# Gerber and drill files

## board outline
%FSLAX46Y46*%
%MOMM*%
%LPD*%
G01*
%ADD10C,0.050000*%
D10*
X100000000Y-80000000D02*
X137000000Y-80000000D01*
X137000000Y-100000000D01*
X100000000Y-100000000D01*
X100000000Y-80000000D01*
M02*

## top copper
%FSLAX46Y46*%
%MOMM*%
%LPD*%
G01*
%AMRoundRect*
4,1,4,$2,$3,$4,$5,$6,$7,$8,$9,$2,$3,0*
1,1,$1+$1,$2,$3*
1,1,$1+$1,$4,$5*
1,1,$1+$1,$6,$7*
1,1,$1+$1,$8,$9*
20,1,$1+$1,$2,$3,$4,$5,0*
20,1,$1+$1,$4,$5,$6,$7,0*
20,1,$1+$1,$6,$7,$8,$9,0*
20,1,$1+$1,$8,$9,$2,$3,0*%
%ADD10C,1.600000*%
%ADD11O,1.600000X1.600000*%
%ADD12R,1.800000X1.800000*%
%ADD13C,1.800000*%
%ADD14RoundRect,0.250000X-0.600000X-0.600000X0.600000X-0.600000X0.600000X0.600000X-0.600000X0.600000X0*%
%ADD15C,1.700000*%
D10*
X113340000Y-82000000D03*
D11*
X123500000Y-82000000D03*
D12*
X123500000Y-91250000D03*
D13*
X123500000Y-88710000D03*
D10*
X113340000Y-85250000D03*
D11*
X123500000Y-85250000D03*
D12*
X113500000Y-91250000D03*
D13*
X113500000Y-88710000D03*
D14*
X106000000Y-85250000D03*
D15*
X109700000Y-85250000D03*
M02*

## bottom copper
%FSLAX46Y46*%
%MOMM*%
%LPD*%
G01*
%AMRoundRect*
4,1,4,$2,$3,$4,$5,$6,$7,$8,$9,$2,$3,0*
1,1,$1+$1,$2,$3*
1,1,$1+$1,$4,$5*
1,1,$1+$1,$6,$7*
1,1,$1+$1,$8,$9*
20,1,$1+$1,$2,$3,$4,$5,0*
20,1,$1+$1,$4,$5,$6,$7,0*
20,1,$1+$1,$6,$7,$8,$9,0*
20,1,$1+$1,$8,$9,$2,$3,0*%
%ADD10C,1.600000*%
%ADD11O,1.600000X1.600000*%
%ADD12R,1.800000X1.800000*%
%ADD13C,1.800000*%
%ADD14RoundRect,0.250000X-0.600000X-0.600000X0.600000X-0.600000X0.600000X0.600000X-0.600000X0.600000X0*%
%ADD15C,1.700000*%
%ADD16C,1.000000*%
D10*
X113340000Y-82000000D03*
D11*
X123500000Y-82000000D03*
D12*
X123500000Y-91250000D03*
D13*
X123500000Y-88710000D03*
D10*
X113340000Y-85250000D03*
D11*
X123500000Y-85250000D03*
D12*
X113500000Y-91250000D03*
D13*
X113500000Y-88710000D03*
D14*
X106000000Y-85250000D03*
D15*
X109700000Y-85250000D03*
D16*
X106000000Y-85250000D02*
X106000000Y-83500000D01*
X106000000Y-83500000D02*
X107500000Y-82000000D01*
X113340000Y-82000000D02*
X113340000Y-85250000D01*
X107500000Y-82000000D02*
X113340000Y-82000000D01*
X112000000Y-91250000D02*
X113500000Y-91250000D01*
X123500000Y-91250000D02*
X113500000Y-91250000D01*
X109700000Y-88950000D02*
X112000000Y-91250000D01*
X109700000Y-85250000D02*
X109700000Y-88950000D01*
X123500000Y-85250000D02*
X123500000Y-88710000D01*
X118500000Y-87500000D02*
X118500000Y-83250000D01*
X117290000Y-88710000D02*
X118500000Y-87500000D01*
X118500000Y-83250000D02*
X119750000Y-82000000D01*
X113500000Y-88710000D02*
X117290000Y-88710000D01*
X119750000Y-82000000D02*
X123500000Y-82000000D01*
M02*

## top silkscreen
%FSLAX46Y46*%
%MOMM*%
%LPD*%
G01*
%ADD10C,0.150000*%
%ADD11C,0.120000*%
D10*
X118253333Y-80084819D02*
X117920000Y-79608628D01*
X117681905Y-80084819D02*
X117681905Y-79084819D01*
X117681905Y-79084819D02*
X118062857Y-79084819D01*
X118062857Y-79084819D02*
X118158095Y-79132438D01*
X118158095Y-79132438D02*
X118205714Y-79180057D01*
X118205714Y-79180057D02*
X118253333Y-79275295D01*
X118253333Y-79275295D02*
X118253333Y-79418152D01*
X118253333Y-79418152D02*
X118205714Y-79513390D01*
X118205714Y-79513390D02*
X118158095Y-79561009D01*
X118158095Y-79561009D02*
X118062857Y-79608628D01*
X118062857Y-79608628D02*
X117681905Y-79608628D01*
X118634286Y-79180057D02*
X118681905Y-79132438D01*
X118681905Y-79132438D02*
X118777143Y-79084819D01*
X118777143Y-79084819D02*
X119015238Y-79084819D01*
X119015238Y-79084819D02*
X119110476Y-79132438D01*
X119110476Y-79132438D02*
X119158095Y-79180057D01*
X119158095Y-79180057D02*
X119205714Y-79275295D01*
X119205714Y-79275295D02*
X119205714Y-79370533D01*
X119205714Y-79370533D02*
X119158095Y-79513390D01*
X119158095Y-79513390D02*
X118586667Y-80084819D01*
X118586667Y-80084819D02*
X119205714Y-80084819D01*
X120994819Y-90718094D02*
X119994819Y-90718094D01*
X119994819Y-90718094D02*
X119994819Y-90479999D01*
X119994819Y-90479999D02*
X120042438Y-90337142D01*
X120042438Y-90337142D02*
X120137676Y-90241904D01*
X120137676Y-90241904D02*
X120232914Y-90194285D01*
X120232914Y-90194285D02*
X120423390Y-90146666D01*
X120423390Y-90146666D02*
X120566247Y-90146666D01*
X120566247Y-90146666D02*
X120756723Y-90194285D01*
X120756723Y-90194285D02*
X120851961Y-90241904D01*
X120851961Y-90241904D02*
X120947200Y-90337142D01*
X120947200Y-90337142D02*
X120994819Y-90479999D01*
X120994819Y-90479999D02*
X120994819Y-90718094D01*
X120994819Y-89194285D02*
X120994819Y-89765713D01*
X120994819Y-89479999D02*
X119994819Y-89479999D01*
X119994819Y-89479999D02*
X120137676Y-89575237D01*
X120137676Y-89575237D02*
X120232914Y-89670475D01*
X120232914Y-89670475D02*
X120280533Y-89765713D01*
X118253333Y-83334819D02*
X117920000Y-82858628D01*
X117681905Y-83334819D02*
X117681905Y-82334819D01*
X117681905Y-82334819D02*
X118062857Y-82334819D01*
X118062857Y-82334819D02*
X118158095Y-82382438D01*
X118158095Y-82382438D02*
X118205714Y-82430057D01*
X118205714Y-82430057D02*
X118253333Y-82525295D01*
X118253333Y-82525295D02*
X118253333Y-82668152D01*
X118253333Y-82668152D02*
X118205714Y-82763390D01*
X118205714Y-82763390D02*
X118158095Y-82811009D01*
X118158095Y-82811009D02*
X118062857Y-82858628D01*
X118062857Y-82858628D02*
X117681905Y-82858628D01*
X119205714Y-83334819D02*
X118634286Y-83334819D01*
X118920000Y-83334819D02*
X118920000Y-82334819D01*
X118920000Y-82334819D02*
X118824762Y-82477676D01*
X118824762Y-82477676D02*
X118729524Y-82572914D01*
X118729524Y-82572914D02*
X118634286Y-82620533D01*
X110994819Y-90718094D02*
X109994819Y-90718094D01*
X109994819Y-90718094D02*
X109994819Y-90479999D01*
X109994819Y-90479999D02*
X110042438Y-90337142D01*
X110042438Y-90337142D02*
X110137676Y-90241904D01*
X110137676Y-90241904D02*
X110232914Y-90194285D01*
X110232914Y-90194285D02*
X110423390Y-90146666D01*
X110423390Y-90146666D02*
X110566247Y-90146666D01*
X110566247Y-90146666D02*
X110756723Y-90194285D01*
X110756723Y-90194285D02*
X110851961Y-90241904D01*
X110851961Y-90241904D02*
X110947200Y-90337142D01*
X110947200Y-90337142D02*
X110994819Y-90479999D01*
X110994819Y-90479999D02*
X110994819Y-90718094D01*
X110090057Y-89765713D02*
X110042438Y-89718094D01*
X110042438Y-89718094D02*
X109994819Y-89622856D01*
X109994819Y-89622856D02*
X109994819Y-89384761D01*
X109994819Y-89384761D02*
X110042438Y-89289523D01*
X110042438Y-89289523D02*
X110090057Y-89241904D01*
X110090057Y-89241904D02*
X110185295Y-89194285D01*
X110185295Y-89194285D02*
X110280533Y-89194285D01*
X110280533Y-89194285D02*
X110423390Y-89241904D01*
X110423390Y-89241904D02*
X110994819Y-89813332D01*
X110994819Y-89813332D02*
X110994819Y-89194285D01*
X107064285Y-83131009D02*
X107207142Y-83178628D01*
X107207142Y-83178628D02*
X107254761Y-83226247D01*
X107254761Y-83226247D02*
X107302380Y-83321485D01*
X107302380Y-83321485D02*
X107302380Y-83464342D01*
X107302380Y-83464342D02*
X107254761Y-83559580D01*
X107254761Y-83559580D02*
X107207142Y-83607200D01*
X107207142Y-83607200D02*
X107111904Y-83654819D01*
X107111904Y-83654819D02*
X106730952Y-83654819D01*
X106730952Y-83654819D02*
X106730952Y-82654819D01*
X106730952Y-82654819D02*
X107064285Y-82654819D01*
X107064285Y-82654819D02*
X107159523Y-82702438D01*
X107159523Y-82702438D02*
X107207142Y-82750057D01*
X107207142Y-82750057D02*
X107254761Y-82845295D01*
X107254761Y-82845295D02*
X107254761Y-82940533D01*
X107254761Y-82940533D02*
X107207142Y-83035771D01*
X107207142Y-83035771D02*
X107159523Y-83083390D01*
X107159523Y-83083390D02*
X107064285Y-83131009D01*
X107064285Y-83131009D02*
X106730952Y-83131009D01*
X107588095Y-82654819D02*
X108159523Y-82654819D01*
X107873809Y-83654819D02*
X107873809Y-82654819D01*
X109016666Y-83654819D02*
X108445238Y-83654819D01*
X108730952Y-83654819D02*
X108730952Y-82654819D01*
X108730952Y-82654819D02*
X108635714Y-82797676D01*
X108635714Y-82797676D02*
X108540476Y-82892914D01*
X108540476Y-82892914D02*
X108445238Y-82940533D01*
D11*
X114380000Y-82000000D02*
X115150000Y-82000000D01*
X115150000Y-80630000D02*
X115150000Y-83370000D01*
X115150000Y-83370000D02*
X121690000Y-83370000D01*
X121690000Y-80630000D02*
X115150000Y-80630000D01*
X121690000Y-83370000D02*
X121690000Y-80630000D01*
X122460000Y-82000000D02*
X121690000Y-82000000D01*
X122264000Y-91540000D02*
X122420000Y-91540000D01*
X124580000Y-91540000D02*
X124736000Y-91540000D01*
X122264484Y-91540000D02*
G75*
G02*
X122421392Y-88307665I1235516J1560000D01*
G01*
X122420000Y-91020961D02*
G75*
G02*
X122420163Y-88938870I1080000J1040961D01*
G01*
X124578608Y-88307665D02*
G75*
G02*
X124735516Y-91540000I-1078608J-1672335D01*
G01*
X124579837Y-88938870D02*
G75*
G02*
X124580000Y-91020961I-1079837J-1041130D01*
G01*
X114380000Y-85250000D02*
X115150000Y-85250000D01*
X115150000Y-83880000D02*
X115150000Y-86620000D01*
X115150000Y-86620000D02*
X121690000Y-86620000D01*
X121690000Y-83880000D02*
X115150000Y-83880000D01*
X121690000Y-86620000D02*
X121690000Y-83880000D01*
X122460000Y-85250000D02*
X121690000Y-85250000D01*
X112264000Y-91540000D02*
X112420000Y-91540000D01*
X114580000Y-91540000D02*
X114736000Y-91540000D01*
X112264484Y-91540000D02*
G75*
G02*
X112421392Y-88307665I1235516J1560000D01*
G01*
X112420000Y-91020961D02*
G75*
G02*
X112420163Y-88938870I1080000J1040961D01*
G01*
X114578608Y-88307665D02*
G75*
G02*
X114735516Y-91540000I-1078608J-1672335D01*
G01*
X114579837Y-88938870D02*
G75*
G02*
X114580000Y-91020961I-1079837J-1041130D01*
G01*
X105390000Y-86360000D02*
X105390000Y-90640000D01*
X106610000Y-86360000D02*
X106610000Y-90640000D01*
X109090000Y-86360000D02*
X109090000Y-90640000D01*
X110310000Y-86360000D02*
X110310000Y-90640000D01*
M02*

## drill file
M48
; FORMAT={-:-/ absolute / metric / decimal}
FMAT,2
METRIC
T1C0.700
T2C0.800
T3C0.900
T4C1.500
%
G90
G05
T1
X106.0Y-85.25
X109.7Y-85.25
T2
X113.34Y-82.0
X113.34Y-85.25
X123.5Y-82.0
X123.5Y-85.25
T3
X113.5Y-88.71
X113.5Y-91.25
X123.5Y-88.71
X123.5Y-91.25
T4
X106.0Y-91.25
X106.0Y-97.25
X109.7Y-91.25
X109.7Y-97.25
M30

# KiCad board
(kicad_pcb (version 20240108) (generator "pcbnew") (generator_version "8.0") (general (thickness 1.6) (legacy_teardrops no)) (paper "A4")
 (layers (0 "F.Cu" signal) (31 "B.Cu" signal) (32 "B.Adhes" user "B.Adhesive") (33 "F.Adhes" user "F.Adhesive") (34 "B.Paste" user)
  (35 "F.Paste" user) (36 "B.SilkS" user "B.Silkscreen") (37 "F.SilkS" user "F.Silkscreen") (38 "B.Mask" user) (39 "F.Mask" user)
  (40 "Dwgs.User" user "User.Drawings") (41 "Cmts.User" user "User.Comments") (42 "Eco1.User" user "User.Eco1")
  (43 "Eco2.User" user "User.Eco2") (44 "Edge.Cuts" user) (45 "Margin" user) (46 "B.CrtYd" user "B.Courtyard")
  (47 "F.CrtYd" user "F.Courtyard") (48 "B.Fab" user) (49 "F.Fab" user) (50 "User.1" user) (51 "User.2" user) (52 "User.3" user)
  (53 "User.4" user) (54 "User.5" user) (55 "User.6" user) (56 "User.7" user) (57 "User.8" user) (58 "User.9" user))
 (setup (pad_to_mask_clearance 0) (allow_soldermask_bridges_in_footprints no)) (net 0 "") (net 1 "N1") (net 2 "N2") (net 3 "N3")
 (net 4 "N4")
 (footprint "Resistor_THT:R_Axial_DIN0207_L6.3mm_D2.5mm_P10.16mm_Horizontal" (layer "F.Cu") (at 113.34 82)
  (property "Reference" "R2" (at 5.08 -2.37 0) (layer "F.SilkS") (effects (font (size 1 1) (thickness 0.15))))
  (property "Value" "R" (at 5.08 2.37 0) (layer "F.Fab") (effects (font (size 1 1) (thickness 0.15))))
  (fp_line (start 1.04 0) (end 1.81 0) (stroke (width 0.12) (type solid)) (layer "F.SilkS"))
  (fp_line (start 1.81 -1.37) (end 1.81 1.37) (stroke (width 0.12) (type solid)) (layer "F.SilkS"))
  (fp_line (start 1.81 1.37) (end 8.35 1.37) (stroke (width 0.12) (type solid)) (layer "F.SilkS"))
  (fp_line (start 8.35 -1.37) (end 1.81 -1.37) (stroke (width 0.12) (type solid)) (layer "F.SilkS"))
  (fp_line (start 8.35 1.37) (end 8.35 -1.37) (stroke (width 0.12) (type solid)) (layer "F.SilkS"))
  (fp_line (start 9.12 0) (end 8.35 0) (stroke (width 0.12) (type solid)) (layer "F.SilkS"))
  (pad "1" thru_hole circle (at 0 0) (size 1.6 1.6) (drill 0.8) (layers "*.Cu" "*.Mask") (remove_unused_layers no) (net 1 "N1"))
  (pad "2" thru_hole oval (at 10.16 0) (size 1.6 1.6) (drill 0.8) (layers "*.Cu" "*.Mask") (remove_unused_layers no) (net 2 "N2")))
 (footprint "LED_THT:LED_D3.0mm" (layer "F.Cu") (at 123.5 91.25 90)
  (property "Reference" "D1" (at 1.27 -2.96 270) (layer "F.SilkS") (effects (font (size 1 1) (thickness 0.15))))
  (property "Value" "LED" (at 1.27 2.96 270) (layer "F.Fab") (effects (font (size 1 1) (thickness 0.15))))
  (fp_line (start -0.29 -1.236) (end -0.29 -1.08) (stroke (width 0.12) (type solid)) (layer "F.SilkS"))
  (fp_line (start -0.29 1.08) (end -0.29 1.236) (stroke (width 0.12) (type solid)) (layer "F.SilkS"))
  (fp_arc (start -0.29 -1.235516) (mid 1.366487 -1.987659) (end 2.942335 -1.078608) (stroke (width 0.12) (type solid)) (layer "F.SilkS"))
  (fp_arc (start 0.229039 -1.08) (mid 1.270117 -1.5) (end 2.31113 -1.079837) (stroke (width 0.12) (type solid)) (layer "F.SilkS"))
  (fp_arc (start 2.942335 1.078608) (mid 1.366487 1.987659) (end -0.29 1.235516) (stroke (width 0.12) (type solid)) (layer "F.SilkS"))
  (fp_arc (start 2.31113 1.079837) (mid 1.270117 1.5) (end 0.229039 1.08) (stroke (width 0.12) (type solid)) (layer "F.SilkS"))
  (pad "1" thru_hole rect (at 0 0 90) (size 1.8 1.8) (drill 0.9) (layers "*.Cu" "*.Mask") (remove_unused_layers no) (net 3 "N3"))
  (pad "2" thru_hole circle (at 2.54 0 90) (size 1.8 1.8) (drill 0.9) (layers "*.Cu" "*.Mask") (remove_unused_layers no) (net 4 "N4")))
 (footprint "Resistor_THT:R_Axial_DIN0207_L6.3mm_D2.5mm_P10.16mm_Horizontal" (layer "F.Cu") (at 113.34 85.25)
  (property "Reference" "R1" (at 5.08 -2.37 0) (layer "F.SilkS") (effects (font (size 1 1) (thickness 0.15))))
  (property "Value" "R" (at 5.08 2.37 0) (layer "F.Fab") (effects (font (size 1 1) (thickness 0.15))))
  (fp_line (start 1.04 0) (end 1.81 0) (stroke (width 0.12) (type solid)) (layer "F.SilkS"))
  (fp_line (start 1.81 -1.37) (end 1.81 1.37) (stroke (width 0.12) (type solid)) (layer "F.SilkS"))
  (fp_line (start 1.81 1.37) (end 8.35 1.37) (stroke (width 0.12) (type solid)) (layer "F.SilkS"))
  (fp_line (start 8.35 -1.37) (end 1.81 -1.37) (stroke (width 0.12) (type solid)) (layer "F.SilkS"))
  (fp_line (start 8.35 1.37) (end 8.35 -1.37) (stroke (width 0.12) (type solid)) (layer "F.SilkS"))
  (fp_line (start 9.12 0) (end 8.35 0) (stroke (width 0.12) (type solid)) (layer "F.SilkS"))
  (pad "1" thru_hole circle (at 0 0) (size 1.6 1.6) (drill 0.8) (layers "*.Cu" "*.Mask") (remove_unused_layers no) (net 1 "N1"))
  (pad "2" thru_hole oval (at 10.16 0) (size 1.6 1.6) (drill 0.8) (layers "*.Cu" "*.Mask") (remove_unused_layers no) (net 4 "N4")))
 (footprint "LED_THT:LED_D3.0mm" (layer "F.Cu") (at 113.5 91.25 90)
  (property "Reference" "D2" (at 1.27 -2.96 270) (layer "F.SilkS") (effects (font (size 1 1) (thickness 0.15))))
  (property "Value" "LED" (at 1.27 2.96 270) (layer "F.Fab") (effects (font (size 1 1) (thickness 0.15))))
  (fp_line (start -0.29 -1.236) (end -0.29 -1.08) (stroke (width 0.12) (type solid)) (layer "F.SilkS"))
  (fp_line (start -0.29 1.08) (end -0.29 1.236) (stroke (width 0.12) (type solid)) (layer "F.SilkS"))
  (fp_arc (start -0.29 -1.235516) (mid 1.366487 -1.987659) (end 2.942335 -1.078608) (stroke (width 0.12) (type solid)) (layer "F.SilkS"))
  (fp_arc (start 0.229039 -1.08) (mid 1.270117 -1.5) (end 2.31113 -1.079837) (stroke (width 0.12) (type solid)) (layer "F.SilkS"))
  (fp_arc (start 2.942335 1.078608) (mid 1.366487 1.987659) (end -0.29 1.235516) (stroke (width 0.12) (type solid)) (layer "F.SilkS"))
  (fp_arc (start 2.31113 1.079837) (mid 1.270117 1.5) (end 0.229039 1.08) (stroke (width 0.12) (type solid)) (layer "F.SilkS"))
  (pad "1" thru_hole rect (at 0 0 90) (size 1.8 1.8) (drill 0.9) (layers "*.Cu" "*.Mask") (remove_unused_layers no) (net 3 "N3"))
  (pad "2" thru_hole circle (at 2.54 0 90) (size 1.8 1.8) (drill 0.9) (layers "*.Cu" "*.Mask") (remove_unused_layers no) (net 2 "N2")))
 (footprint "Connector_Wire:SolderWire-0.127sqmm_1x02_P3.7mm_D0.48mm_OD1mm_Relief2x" (layer "F.Cu") (at 106 85.25)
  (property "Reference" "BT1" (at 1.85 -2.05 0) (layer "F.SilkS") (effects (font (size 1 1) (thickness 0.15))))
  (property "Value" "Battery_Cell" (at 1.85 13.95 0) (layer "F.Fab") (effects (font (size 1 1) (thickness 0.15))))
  (fp_line (start -0.61 1.11) (end -0.61 5.39) (stroke (width 0.12) (type solid)) (layer "F.SilkS"))
  (fp_line (start 0.61 1.11) (end 0.61 5.39) (stroke (width 0.12) (type solid)) (layer "F.SilkS"))
  (fp_line (start 3.09 1.11) (end 3.09 5.39) (stroke (width 0.12) (type solid)) (layer "F.SilkS"))
  (fp_line (start 4.31 1.11) (end 4.31 5.39) (stroke (width 0.12) (type solid)) (layer "F.SilkS"))
  (pad "" np_thru_hole circle (at 0 6) (size 1.5 1.5) (drill 1.5) (layers "*.Cu" "*.Mask"))
  (pad "" np_thru_hole circle (at 0 12) (size 1.5 1.5) (drill 1.5) (layers "*.Cu" "*.Mask"))
  (pad "" np_thru_hole circle (at 3.7 6) (size 1.5 1.5) (drill 1.5) (layers "*.Cu" "*.Mask"))
  (pad "" np_thru_hole circle (at 3.7 12) (size 1.5 1.5) (drill 1.5) (layers "*.Cu" "*.Mask"))
  (pad "1" thru_hole roundrect (at 0 0) (size 1.7 1.7) (drill 0.7) (layers "*.Cu" "*.Mask") (remove_unused_layers no)
   (roundrect_rratio 0.147059) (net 1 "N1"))
  (pad "2" thru_hole circle (at 3.7 0) (size 1.7 1.7) (drill 0.7) (layers "*.Cu" "*.Mask") (remove_unused_layers no) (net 3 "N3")))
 (gr_rect (start 100 80) (end 137 100) (stroke (width 0.05) (type default)) (fill none) (layer "Edge.Cuts"))
 (segment (start 106 85.25) (end 106 83.5) (width 1) (layer "B.Cu") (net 1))
 (segment (start 106 83.5) (end 107.5 82) (width 1) (layer "B.Cu") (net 1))
 (segment (start 113.34 82) (end 113.34 85.25) (width 1) (layer "B.Cu") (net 1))
 (segment (start 107.5 82) (end 113.34 82) (width 1) (layer "B.Cu") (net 1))
 (segment (start 112 91.25) (end 113.5 91.25) (width 1) (layer "B.Cu") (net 3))
 (segment (start 123.5 91.25) (end 113.5 91.25) (width 1) (layer "B.Cu") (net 3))
 (segment (start 109.7 88.95) (end 112 91.25) (width 1) (layer "B.Cu") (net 3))
 (segment (start 109.7 85.25) (end 109.7 88.95) (width 1) (layer "B.Cu") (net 3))
 (segment (start 123.5 85.25) (end 123.5 88.71) (width 1) (layer "B.Cu") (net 4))
 (segment (start 118.5 87.5) (end 118.5 83.25) (width 1) (layer "B.Cu") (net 2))
 (segment (start 117.29 88.71) (end 118.5 87.5) (width 1) (layer "B.Cu") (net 2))
 (segment (start 118.5 83.25) (end 119.75 82) (width 1) (layer "B.Cu") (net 2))
 (segment (start 113.5 88.71) (end 117.29 88.71) (width 1) (layer "B.Cu") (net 2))
 (segment (start 119.75 82) (end 123.5 82) (width 1) (layer "B.Cu") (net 2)))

